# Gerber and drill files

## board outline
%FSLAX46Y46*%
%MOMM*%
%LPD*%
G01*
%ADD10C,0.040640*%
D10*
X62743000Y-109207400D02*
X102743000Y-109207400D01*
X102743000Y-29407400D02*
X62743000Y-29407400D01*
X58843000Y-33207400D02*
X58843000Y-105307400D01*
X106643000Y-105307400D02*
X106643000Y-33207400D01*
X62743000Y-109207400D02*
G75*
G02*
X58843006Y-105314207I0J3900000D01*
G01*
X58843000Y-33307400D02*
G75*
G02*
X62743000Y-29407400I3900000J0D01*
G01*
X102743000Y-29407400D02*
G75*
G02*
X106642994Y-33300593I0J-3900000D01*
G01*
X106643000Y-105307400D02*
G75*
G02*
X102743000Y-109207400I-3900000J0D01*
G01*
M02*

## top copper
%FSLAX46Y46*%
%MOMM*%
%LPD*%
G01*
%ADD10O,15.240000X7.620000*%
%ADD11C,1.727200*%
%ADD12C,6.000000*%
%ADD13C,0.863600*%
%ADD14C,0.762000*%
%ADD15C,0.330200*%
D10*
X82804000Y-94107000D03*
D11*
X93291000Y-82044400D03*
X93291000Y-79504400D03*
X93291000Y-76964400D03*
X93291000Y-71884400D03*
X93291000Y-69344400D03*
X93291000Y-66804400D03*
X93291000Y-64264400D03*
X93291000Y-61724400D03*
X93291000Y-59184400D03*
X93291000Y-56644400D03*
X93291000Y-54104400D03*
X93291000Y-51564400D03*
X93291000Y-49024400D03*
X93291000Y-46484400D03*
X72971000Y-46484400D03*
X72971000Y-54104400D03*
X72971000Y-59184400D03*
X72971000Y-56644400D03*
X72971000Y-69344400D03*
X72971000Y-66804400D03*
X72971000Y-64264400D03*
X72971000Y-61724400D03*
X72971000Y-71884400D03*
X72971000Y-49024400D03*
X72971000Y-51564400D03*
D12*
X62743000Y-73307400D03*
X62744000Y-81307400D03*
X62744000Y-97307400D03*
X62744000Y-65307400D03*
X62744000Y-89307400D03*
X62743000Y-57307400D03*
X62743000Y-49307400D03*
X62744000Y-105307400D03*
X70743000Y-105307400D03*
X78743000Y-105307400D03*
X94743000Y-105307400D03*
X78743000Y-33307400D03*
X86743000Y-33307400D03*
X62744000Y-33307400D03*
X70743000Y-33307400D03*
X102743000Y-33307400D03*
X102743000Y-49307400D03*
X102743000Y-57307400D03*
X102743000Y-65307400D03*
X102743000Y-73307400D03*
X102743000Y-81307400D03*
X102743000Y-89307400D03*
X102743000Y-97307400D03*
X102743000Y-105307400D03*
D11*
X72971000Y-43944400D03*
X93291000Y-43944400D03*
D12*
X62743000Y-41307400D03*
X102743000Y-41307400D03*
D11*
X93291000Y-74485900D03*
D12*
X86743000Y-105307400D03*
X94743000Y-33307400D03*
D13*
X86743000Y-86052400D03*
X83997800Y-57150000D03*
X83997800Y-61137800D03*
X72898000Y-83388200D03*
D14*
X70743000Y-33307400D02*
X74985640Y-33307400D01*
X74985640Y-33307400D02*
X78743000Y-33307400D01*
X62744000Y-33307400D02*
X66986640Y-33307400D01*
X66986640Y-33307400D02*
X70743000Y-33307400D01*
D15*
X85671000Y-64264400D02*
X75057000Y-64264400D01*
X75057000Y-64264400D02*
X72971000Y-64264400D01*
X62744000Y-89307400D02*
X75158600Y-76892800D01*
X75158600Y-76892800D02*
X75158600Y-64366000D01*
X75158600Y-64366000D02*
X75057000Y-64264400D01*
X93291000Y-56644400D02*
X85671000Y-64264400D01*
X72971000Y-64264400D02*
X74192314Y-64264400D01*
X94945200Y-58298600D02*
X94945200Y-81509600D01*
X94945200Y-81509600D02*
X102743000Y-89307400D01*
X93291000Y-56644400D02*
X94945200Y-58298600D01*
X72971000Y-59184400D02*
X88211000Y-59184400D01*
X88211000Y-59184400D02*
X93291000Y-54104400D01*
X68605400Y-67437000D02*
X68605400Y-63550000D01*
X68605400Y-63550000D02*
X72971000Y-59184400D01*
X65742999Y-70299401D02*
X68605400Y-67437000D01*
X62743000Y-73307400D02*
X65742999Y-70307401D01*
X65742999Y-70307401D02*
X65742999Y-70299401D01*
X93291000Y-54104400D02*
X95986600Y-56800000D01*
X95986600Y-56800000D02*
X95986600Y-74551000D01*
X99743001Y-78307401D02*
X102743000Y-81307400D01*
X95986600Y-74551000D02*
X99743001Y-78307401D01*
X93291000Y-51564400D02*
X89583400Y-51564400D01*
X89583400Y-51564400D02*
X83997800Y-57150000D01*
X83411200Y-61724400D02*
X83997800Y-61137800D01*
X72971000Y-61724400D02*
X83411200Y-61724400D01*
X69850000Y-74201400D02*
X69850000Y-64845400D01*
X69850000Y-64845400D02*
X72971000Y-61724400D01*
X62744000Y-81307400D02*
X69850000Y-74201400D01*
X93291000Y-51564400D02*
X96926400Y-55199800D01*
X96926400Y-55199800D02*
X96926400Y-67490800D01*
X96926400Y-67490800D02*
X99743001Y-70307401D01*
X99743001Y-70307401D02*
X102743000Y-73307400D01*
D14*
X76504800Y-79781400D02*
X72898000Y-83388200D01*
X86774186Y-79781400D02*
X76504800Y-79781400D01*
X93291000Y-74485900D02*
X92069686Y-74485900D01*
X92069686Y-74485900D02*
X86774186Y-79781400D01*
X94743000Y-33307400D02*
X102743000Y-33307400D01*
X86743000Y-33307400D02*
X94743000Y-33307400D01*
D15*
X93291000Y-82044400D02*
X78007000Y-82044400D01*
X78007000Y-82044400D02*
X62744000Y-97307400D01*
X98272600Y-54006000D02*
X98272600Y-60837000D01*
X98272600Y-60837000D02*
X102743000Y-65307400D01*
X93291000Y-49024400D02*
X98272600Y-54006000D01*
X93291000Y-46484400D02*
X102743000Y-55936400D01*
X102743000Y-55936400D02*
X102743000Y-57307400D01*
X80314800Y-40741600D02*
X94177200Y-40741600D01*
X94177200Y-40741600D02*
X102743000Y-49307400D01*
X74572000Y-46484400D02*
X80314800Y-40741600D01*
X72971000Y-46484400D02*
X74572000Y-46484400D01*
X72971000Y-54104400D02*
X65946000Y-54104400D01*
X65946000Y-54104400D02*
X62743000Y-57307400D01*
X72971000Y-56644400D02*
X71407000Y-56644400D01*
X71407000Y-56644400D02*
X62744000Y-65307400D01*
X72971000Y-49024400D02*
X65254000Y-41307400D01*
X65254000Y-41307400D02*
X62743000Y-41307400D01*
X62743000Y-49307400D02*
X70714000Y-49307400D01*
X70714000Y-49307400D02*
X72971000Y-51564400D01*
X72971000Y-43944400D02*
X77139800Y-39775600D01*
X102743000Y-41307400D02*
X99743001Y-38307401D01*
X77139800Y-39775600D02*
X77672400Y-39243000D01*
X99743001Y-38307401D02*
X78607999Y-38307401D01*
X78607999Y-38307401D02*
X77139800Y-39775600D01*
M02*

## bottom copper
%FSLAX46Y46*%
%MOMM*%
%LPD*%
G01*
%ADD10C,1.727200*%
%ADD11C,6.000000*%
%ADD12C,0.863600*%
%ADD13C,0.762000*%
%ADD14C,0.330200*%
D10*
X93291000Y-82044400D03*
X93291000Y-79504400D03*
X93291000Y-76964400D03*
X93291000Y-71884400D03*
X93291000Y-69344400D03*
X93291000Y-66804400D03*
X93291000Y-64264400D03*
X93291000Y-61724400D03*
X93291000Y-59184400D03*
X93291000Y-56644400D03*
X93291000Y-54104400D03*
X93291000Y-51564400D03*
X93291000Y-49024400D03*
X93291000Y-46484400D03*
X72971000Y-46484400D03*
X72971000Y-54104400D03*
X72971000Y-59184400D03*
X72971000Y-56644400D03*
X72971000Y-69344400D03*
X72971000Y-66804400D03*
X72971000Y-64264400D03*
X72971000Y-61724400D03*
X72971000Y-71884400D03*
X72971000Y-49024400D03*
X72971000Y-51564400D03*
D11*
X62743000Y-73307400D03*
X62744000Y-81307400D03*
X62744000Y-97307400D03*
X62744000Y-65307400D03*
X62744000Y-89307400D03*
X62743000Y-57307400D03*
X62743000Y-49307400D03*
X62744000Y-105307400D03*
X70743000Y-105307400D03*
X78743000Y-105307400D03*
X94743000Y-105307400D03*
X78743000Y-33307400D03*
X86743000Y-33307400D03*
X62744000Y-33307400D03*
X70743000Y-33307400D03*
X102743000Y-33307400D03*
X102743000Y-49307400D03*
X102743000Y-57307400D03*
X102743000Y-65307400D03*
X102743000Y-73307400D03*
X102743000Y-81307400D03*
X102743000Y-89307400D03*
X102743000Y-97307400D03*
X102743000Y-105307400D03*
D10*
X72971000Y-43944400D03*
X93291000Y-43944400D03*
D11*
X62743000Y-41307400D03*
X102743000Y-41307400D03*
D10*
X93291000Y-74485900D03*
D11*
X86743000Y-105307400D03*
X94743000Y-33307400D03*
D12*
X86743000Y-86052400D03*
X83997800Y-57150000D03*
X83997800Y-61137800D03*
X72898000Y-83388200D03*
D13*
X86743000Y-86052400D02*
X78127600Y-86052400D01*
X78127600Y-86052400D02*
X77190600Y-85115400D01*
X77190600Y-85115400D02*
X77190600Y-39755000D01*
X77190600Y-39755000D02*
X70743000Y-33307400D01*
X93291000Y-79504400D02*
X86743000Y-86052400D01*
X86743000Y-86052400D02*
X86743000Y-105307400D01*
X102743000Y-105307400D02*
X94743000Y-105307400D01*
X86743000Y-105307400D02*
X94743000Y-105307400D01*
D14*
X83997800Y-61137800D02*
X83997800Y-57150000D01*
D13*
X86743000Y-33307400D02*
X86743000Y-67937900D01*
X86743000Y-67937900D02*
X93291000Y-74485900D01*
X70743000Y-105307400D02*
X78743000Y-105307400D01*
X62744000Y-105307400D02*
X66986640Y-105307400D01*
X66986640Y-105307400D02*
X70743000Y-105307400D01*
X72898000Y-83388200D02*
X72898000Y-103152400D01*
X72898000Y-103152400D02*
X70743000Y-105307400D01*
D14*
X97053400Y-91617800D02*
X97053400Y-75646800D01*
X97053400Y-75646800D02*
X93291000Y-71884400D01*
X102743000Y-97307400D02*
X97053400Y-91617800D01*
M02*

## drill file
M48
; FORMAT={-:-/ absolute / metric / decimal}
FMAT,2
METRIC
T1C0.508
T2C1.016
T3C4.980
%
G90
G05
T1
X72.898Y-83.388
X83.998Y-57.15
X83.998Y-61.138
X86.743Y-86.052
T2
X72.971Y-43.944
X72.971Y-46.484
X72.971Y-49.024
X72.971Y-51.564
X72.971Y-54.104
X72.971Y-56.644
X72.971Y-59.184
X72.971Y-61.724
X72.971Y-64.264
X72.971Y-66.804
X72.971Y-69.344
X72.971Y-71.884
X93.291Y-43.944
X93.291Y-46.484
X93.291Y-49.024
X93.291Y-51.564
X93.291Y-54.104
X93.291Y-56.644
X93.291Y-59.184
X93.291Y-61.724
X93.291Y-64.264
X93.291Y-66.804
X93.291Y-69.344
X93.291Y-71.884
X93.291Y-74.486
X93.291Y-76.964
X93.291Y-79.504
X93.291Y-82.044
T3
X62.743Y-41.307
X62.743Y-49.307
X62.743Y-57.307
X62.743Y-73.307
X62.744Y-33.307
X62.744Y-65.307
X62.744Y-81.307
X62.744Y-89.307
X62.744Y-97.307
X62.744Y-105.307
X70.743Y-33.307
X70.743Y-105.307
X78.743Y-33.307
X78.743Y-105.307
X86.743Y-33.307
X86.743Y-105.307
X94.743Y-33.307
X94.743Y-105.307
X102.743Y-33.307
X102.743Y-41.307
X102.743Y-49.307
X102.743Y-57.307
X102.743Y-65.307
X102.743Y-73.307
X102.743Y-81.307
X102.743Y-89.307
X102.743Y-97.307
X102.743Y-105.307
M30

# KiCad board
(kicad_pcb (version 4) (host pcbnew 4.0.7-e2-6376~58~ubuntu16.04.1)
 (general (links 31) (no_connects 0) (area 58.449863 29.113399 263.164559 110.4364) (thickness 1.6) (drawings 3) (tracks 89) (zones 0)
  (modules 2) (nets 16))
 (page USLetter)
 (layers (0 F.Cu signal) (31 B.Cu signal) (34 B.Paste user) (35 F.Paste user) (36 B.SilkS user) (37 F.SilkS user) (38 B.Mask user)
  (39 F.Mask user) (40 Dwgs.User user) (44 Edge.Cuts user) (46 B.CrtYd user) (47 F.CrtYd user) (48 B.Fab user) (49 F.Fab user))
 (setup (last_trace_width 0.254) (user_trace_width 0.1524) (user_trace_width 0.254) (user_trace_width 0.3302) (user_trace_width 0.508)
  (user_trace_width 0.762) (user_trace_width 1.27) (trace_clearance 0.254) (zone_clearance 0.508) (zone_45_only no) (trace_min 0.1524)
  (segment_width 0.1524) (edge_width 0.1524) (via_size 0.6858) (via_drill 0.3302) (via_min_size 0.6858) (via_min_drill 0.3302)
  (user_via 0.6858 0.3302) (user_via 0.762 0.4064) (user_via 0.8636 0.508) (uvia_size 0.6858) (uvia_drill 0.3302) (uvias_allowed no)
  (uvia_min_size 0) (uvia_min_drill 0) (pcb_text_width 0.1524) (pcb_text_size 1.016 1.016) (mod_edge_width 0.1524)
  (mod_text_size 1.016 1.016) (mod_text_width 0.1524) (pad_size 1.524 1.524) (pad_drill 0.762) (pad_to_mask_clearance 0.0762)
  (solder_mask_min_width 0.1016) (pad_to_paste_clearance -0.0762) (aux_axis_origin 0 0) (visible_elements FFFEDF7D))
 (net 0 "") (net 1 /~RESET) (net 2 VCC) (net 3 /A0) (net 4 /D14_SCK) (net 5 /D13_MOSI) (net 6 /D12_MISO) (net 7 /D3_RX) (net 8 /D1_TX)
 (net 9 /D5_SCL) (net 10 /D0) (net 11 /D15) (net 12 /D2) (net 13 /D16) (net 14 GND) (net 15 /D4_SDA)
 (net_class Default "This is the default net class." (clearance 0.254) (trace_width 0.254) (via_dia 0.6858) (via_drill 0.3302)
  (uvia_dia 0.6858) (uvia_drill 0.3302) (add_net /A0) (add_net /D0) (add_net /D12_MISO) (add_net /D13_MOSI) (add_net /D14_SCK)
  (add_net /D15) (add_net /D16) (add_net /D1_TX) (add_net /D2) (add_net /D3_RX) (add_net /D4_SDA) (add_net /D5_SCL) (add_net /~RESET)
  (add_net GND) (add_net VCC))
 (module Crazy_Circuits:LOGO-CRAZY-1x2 (layer F.Cu) (at 82.804 98.044)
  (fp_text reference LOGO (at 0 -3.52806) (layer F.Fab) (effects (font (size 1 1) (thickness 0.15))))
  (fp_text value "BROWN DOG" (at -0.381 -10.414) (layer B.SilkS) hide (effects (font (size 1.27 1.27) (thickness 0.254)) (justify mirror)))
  (pad BG smd oval (at 0 -3.937) (size 15.24 7.62) (layers F.Cu)))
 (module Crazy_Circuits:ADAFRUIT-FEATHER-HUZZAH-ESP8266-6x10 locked (layer F.Cu) (at 62.743 65.3074)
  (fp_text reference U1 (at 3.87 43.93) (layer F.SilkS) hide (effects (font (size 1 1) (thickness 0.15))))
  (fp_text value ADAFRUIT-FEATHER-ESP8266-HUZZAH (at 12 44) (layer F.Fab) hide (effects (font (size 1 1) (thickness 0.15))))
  (fp_line (start 0 43.9) (end 40 43.9) (layer Edge.Cuts) (width 0.04064))
  (fp_line (start 40 -35.9) (end 0 -35.9) (layer Edge.Cuts) (width 0.04064))
  (fp_line (start -3.9 -32.1) (end -3.9 40) (layer Edge.Cuts) (width 0.04064))
  (fp_line (start 43.9 40) (end 43.9 -32.1) (layer Edge.Cuts) (width 0.04064))
  (fp_arc (start 0 40) (end 0 43.9) (angle 89.9) (layer Edge.Cuts) (width 0.04064))
  (fp_arc (start 0 -32) (end -3.9 -32) (angle 90) (layer Edge.Cuts) (width 0.04064))
  (fp_arc (start 40 -32) (end 40 -35.9) (angle 89.9) (layer Edge.Cuts) (width 0.04064))
  (fp_arc (start 40 40) (end 43.9 40) (angle 90) (layer Edge.Cuts) (width 0.04064))
  (pad 1 thru_hole circle (at 30.548 16.737 180) (size 1.7272 1.7272) (drill 1.016) (layers *.Cu *.Mask F.SilkS) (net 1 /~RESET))
  (pad 3V thru_hole circle (at 30.548 14.197 180) (size 1.7272 1.7272) (drill 1.016) (layers *.Cu *.Mask F.SilkS) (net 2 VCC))
  (pad NC thru_hole circle (at 30.548 11.657 180) (size 1.7272 1.7272) (drill 1.016) (layers *.Cu *.Mask F.SilkS))
  (pad 2 thru_hole circle (at 30.548 6.577 180) (size 1.7272 1.7272) (drill 1.016) (layers *.Cu *.Mask F.SilkS) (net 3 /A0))
  (pad NC thru_hole circle (at 30.548 4.037 180) (size 1.7272 1.7272) (drill 1.016) (layers *.Cu *.Mask F.SilkS))
  (pad NC thru_hole circle (at 30.548 1.497 180) (size 1.7272 1.7272) (drill 1.016) (layers *.Cu *.Mask F.SilkS))
  (pad NC thru_hole circle (at 30.548 -1.043 180) (size 1.7272 1.7272) (drill 1.016) (layers *.Cu *.Mask F.SilkS))
  (pad NC thru_hole circle (at 30.548 -3.583 180) (size 1.7272 1.7272) (drill 1.016) (layers *.Cu *.Mask F.SilkS))
  (pad NC thru_hole circle (at 30.548 -6.123 180) (size 1.7272 1.7272) (drill 1.016) (layers *.Cu *.Mask F.SilkS))
  (pad 5 thru_hole circle (at 30.548 -8.663 180) (size 1.7272 1.7272) (drill 1.016) (layers *.Cu *.Mask F.SilkS) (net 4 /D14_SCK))
  (pad 7 thru_hole circle (at 30.548 -11.203 180) (size 1.7272 1.7272) (drill 1.016) (layers *.Cu *.Mask F.SilkS) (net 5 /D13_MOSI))
  (pad 6 thru_hole circle (at 30.548 -13.743 180) (size 1.7272 1.7272) (drill 1.016) (layers *.Cu *.Mask F.SilkS) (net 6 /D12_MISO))
  (pad 15 thru_hole circle (at 30.548 -16.283 180) (size 1.7272 1.7272) (drill 1.016) (layers *.Cu *.Mask F.SilkS) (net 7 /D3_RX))
  (pad 16 thru_hole circle (at 30.548 -18.823 180) (size 1.7272 1.7272) (drill 1.016) (layers *.Cu *.Mask F.SilkS) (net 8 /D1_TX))
  (pad 14 thru_hole circle (at 10.228 -18.823 180) (size 1.7272 1.7272) (drill 1.016) (layers *.Cu *.Mask F.SilkS) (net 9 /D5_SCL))
  (pad 12 thru_hole circle (at 10.228 -11.203 180) (size 1.7272 1.7272) (drill 1.016) (layers *.Cu *.Mask F.SilkS) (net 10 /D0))
  (pad 7 thru_hole circle (at 10.228 -6.123 180) (size 1.7272 1.7272) (drill 1.016) (layers *.Cu *.Mask F.SilkS) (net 5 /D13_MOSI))
  (pad 10 thru_hole circle (at 10.228 -8.663 180) (size 1.7272 1.7272) (drill 1.016) (layers *.Cu *.Mask F.SilkS) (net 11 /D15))
  (pad EN thru_hole circle (at 10.228 4.037 180) (size 1.7272 1.7272) (drill 1.016) (layers *.Cu *.Mask F.SilkS))
  (pad USB thru_hole circle (at 10.228 1.497 180) (size 1.7272 1.7272) (drill 1.016) (layers *.Cu *.Mask F.SilkS))
  (pad 5 thru_hole circle (at 10.228 -1.043 180) (size 1.7272 1.7272) (drill 1.016) (layers *.Cu *.Mask F.SilkS) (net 4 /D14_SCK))
  (pad 6 thru_hole circle (at 10.228 -3.583 180) (size 1.7272 1.7272) (drill 1.016) (layers *.Cu *.Mask F.SilkS) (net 6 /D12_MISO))
  (pad VBAT thru_hole circle (at 10.228 6.577 180) (size 1.7272 1.7272) (drill 1.016) (layers *.Cu *.Mask F.SilkS))
  (pad 11 thru_hole circle (at 10.228 -16.283 180) (size 1.7272 1.7272) (drill 1.016) (layers *.Cu *.Mask F.SilkS) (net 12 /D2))
  (pad 4 thru_hole circle (at 10.228 -13.743 180) (size 1.7272 1.7272) (drill 1.016) (layers *.Cu *.Mask F.SilkS) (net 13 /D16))
  (pad 7 thru_hole circle (at 0 8 90) (size 6 6) (drill 4.98) (layers *.Cu *.Mask) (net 5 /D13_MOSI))
  (pad 6 thru_hole circle (at 0.001 16 90) (size 6 6) (drill 4.98) (layers *.Cu *.Mask) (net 6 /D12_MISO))
  (pad 1 thru_hole circle (at 0.001 32 90) (size 6 6) (drill 4.98) (layers *.Cu *.Mask) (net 1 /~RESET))
  (pad 10 thru_hole circle (at 0.001 0 90) (size 6 6) (drill 4.98) (layers *.Cu *.Mask) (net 11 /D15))
  (pad 5 thru_hole circle (at 0.001 24 90) (size 6 6) (drill 4.98) (layers *.Cu *.Mask) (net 4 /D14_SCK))
  (pad 12 thru_hole circle (at 0 -8 90) (size 6 6) (drill 4.98) (layers *.Cu *.Mask) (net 10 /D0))
  (pad 4 thru_hole circle (at 0 -16 90) (size 6 6) (drill 4.98) (layers *.Cu *.Mask) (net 13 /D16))
  (pad GND thru_hole circle (at 0.001 40 90) (size 6 6) (drill 4.98) (layers *.Cu *.Mask) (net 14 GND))
  (pad GND thru_hole circle (at 8 40 90) (size 6 6) (drill 4.98) (layers *.Cu *.Mask) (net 14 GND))
  (pad GND thru_hole circle (at 16 40 90) (size 6 6) (drill 4.98) (layers *.Cu *.Mask) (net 14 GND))
  (pad 3V thru_hole circle (at 32 40 90) (size 6 6) (drill 4.98) (layers *.Cu *.Mask) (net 2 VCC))
  (pad 3V thru_hole circle (at 16 -32 90) (size 6 6) (drill 4.98) (layers *.Cu *.Mask) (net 2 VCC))
  (pad GND thru_hole circle (at 24 -32 90) (size 6 6) (drill 4.98) (layers *.Cu *.Mask) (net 14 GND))
  (pad 3V thru_hole circle (at 0.001 -32 90) (size 6 6) (drill 4.98) (layers *.Cu *.Mask) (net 2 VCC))
  (pad 3V thru_hole circle (at 8 -32 90) (size 6 6) (drill 4.98) (layers *.Cu *.Mask) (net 2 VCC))
  (pad GND thru_hole circle (at 40 -32 90) (size 6 6) (drill 4.98) (layers *.Cu *.Mask) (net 14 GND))
  (pad 14 thru_hole circle (at 40 -16 90) (size 6 6) (drill 4.98) (layers *.Cu *.Mask) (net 9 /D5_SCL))
  (pad 16 thru_hole circle (at 40 -8 90) (size 6 6) (drill 4.98) (layers *.Cu *.Mask) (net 8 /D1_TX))
  (pad 15 thru_hole circle (at 40 0 90) (size 6 6) (drill 4.98) (layers *.Cu *.Mask) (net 7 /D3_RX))
  (pad 6 thru_hole circle (at 40 8 90) (size 6 6) (drill 4.98) (layers *.Cu *.Mask) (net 6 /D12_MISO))
  (pad 7 thru_hole circle (at 40 16 90) (size 6 6) (drill 4.98) (layers *.Cu *.Mask) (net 5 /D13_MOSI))
  (pad 5 thru_hole circle (at 40 24 90) (size 6 6) (drill 4.98) (layers *.Cu *.Mask) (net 4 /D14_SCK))
  (pad 2 thru_hole circle (at 40 32 90) (size 6 6) (drill 4.98) (layers *.Cu *.Mask) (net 3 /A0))
  (pad 3V thru_hole circle (at 40 40 90) (size 6 6) (drill 4.98) (layers *.Cu *.Mask) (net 2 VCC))
  (pad 13 thru_hole circle (at 10.228 -21.363 180) (size 1.7272 1.7272) (drill 1.016) (layers *.Cu *.Mask F.SilkS) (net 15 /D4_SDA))
  (pad 3 thru_hole circle (at 30.548 -21.363 180) (size 1.7272 1.7272) (drill 1.016) (layers *.Cu *.Mask F.SilkS))
  (pad 11 thru_hole circle (at 0 -24 90) (size 6 6) (drill 4.98) (layers *.Cu *.Mask) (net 12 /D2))
  (pad 13 thru_hole circle (at 40 -24 90) (size 6 6) (drill 4.98) (layers *.Cu *.Mask) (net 15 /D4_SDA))
  (pad GND thru_hole circle (at 30.548 9.1785 180) (size 1.7272 1.7272) (drill 1.016) (layers *.Cu *.Mask F.SilkS) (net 14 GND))
  (pad 3V thru_hole circle (at 24 40 90) (size 6 6) (drill 4.98) (layers *.Cu *.Mask) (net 2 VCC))
  (pad GND thru_hole circle (at 32 -32 90) (size 6 6) (drill 4.98) (layers *.Cu *.Mask) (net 14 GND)))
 (segment (start 86.743 86.0524) (end 78.1276 86.0524) (width 0.762) (layer B.Cu) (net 2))
 (segment (start 78.1276 86.0524) (end 77.1906 85.1154) (width 0.762) (layer B.Cu) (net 2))
 (segment (start 77.1906 85.1154) (end 77.1906 39.755) (width 0.762) (layer B.Cu) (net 2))
 (segment (start 77.1906 39.755) (end 70.743 33.3074) (width 0.762) (layer B.Cu) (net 2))
 (via (at 86.743 86.0524) (size 0.8636) (drill 0.508) (layers F.Cu B.Cu) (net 2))
 (segment (start 93.291 79.5044) (end 86.743 86.0524) (width 0.762) (layer B.Cu) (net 2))
 (segment (start 86.743 86.0524) (end 86.743 105.3074) (width 0.762) (layer B.Cu) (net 2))
 (segment (start 102.743 105.3074) (end 94.743 105.3074) (width 0.762) (layer B.Cu) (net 2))
 (segment (start 86.743 105.3074) (end 94.743 105.3074) (width 0.762) (layer B.Cu) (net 2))
 (segment (start 70.743 33.3074) (end 74.98564 33.3074) (width 0.762) (layer F.Cu) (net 2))
 (segment (start 74.98564 33.3074) (end 78.743 33.3074) (width 0.762) (layer F.Cu) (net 2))
 (segment (start 62.744 33.3074) (end 66.98664 33.3074) (width 0.762) (layer F.Cu) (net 2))
 (segment (start 66.98664 33.3074) (end 70.743 33.3074) (width 0.762) (layer F.Cu) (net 2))
 (segment (start 85.671 64.2644) (end 75.057 64.2644) (width 0.3302) (layer F.Cu) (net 4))
 (segment (start 75.057 64.2644) (end 72.971 64.2644) (width 0.3302) (layer F.Cu) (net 4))
 (segment (start 62.744 89.3074) (end 75.1586 76.8928) (width 0.3302) (layer F.Cu) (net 4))
 (segment (start 75.1586 76.8928) (end 75.1586 64.366) (width 0.3302) (layer F.Cu) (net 4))
 (segment (start 75.1586 64.366) (end 75.057 64.2644) (width 0.3302) (layer F.Cu) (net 4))
 (segment (start 93.291 56.6444) (end 85.671 64.2644) (width 0.3302) (layer F.Cu) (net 4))
 (segment (start 72.971 64.2644) (end 74.192314 64.2644) (width 0.3302) (layer F.Cu) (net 4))
 (segment (start 94.9452 58.2986) (end 94.9452 81.5096) (width 0.3302) (layer F.Cu) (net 4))
 (segment (start 94.9452 81.5096) (end 102.743 89.3074) (width 0.3302) (layer F.Cu) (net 4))
 (segment (start 93.291 56.6444) (end 94.9452 58.2986) (width 0.3302) (layer F.Cu) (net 4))
 (segment (start 72.971 59.1844) (end 88.211 59.1844) (width 0.3302) (layer F.Cu) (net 5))
 (segment (start 88.211 59.1844) (end 93.291 54.1044) (width 0.3302) (layer F.Cu) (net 5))
 (segment (start 68.6054 67.437) (end 68.6054 63.55) (width 0.3302) (layer F.Cu) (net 5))
 (segment (start 68.6054 63.55) (end 72.971 59.1844) (width 0.3302) (layer F.Cu) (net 5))
 (segment (start 65.742999 70.299401) (end 68.6054 67.437) (width 0.3302) (layer F.Cu) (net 5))
 (segment (start 62.743 73.3074) (end 65.742999 70.307401) (width 0.3302) (layer F.Cu) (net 5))
 (segment (start 65.742999 70.307401) (end 65.742999 70.299401) (width 0.3302) (layer F.Cu) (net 5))
 (segment (start 93.291 54.1044) (end 95.9866 56.8) (width 0.3302) (layer F.Cu) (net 5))
 (segment (start 95.9866 56.8) (end 95.9866 74.551) (width 0.3302) (layer F.Cu) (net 5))
 (segment (start 99.743001 78.307401) (end 102.743 81.3074) (width 0.3302) (layer F.Cu) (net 5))
 (segment (start 95.9866 74.551) (end 99.743001 78.307401) (width 0.3302) (layer F.Cu) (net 5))
 (segment (start 93.291 51.5644) (end 89.5834 51.5644) (width 0.3302) (layer F.Cu) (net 6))
 (segment (start 89.5834 51.5644) (end 83.9978 57.15) (width 0.3302) (layer F.Cu) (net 6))
 (via (at 83.9978 57.15) (size 0.8636) (drill 0.508) (layers F.Cu B.Cu) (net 6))
 (segment (start 83.9978 61.1378) (end 83.9978 57.15) (width 0.3302) (layer B.Cu) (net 6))
 (segment (start 83.4112 61.7244) (end 83.9978 61.1378) (width 0.3302) (layer F.Cu) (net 6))
 (via (at 83.9978 61.1378) (size 0.8636) (drill 0.508) (layers F.Cu B.Cu) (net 6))
 (segment (start 72.971 61.7244) (end 83.4112 61.7244) (width 0.3302) (layer F.Cu) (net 6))
 (segment (start 69.85 74.2014) (end 69.85 64.8454) (width 0.3302) (layer F.Cu) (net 6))
 (segment (start 69.85 64.8454) (end 72.971 61.7244) (width 0.3302) (layer F.Cu) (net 6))
 (segment (start 62.744 81.3074) (end 69.85 74.2014) (width 0.3302) (layer F.Cu) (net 6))
 (segment (start 93.291 51.5644) (end 96.9264 55.1998) (width 0.3302) (layer F.Cu) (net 6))
 (segment (start 96.9264 55.1998) (end 96.9264 67.4908) (width 0.3302) (layer F.Cu) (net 6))
 (segment (start 96.9264 67.4908) (end 99.743001 70.307401) (width 0.3302) (layer F.Cu) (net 6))
 (segment (start 99.743001 70.307401) (end 102.743 73.3074) (width 0.3302) (layer F.Cu) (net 6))
 (segment (start 86.743 33.3074) (end 86.743 67.9379) (width 0.762) (layer B.Cu) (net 14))
 (segment (start 86.743 67.9379) (end 93.291 74.4859) (width 0.762) (layer B.Cu) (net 14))
 (segment (start 70.743 105.3074) (end 78.743 105.3074) (width 0.762) (layer B.Cu) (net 14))
 (segment (start 62.744 105.3074) (end 66.98664 105.3074) (width 0.762) (layer B.Cu) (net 14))
 (segment (start 66.98664 105.3074) (end 70.743 105.3074) (width 0.762) (layer B.Cu) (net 14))
 (segment (start 72.898 83.3882) (end 72.898 103.1524) (width 0.762) (layer B.Cu) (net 14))
 (segment (start 72.898 103.1524) (end 70.743 105.3074) (width 0.762) (layer B.Cu) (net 14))
 (via (at 72.898 83.3882) (size 0.8636) (drill 0.508) (layers F.Cu B.Cu) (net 14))
 (segment (start 76.5048 79.7814) (end 72.898 83.3882) (width 0.762) (layer F.Cu) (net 14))
 (segment (start 86.774186 79.7814) (end 76.5048 79.7814) (width 0.762) (layer F.Cu) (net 14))
 (segment (start 93.291 74.4859) (end 92.069686 74.4859) (width 0.762) (layer F.Cu) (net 14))
 (segment (start 92.069686 74.4859) (end 86.774186 79.7814) (width 0.762) (layer F.Cu) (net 14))
 (segment (start 94.743 33.3074) (end 102.743 33.3074) (width 0.762) (layer F.Cu) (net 14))
 (segment (start 86.743 33.3074) (end 94.743 33.3074) (width 0.762) (layer F.Cu) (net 14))
 (segment (start 93.291 82.0444) (end 78.007 82.0444) (width 0.3302) (layer F.Cu) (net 1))
 (segment (start 78.007 82.0444) (end 62.744 97.3074) (width 0.3302) (layer F.Cu) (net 1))
 (segment (start 97.0534 91.6178) (end 97.0534 75.6468) (width 0.3302) (layer B.Cu) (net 3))
 (segment (start 97.0534 75.6468) (end 93.291 71.8844) (width 0.3302) (layer B.Cu) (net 3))
 (segment (start 102.743 97.3074) (end 97.0534 91.6178) (width 0.3302) (layer B.Cu) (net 3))
 (segment (start 98.2726 54.006) (end 98.2726 60.837) (width 0.3302) (layer F.Cu) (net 7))
 (segment (start 98.2726 60.837) (end 102.743 65.3074) (width 0.3302) (layer F.Cu) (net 7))
 (segment (start 93.291 49.0244) (end 98.2726 54.006) (width 0.3302) (layer F.Cu) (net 7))
 (segment (start 93.291 46.4844) (end 102.743 55.9364) (width 0.3302) (layer F.Cu) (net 8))
 (segment (start 102.743 55.9364) (end 102.743 57.3074) (width 0.3302) (layer F.Cu) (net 8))
 (segment (start 80.3148 40.7416) (end 94.1772 40.7416) (width 0.3302) (layer F.Cu) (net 9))
 (segment (start 94.1772 40.7416) (end 102.743 49.3074) (width 0.3302) (layer F.Cu) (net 9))
 (segment (start 74.572 46.4844) (end 80.3148 40.7416) (width 0.3302) (layer F.Cu) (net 9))
 (segment (start 72.971 46.4844) (end 74.572 46.4844) (width 0.3302) (layer F.Cu) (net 9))
 (segment (start 72.971 54.1044) (end 65.946 54.1044) (width 0.3302) (layer F.Cu) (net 10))
 (segment (start 65.946 54.1044) (end 62.743 57.3074) (width 0.3302) (layer F.Cu) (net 10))
 (segment (start 72.971 56.6444) (end 71.407 56.6444) (width 0.3302) (layer F.Cu) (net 11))
 (segment (start 71.407 56.6444) (end 62.744 65.3074) (width 0.3302) (layer F.Cu) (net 11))
 (segment (start 72.971 49.0244) (end 65.254 41.3074) (width 0.3302) (layer F.Cu) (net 12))
 (segment (start 65.254 41.3074) (end 62.743 41.3074) (width 0.3302) (layer F.Cu) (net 12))
 (segment (start 62.743 49.3074) (end 70.714 49.3074) (width 0.3302) (layer F.Cu) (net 13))
 (segment (start 70.714 49.3074) (end 72.971 51.5644) (width 0.3302) (layer F.Cu) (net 13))
 (segment (start 72.971 43.9444) (end 77.1398 39.7756) (width 0.3302) (layer F.Cu) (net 15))
 (segment (start 102.743 41.3074) (end 99.743001 38.307401) (width 0.3302) (layer F.Cu) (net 15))
 (segment (start 77.1398 39.7756) (end 77.6724 39.243) (width 0.3302) (layer F.Cu) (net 15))
 (segment (start 99.743001 38.307401) (end 78.607999 38.307401) (width 0.3302) (layer F.Cu) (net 15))
 (segment (start 78.607999 38.307401) (end 77.1398 39.7756) (width 0.3302) (layer F.Cu) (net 15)))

